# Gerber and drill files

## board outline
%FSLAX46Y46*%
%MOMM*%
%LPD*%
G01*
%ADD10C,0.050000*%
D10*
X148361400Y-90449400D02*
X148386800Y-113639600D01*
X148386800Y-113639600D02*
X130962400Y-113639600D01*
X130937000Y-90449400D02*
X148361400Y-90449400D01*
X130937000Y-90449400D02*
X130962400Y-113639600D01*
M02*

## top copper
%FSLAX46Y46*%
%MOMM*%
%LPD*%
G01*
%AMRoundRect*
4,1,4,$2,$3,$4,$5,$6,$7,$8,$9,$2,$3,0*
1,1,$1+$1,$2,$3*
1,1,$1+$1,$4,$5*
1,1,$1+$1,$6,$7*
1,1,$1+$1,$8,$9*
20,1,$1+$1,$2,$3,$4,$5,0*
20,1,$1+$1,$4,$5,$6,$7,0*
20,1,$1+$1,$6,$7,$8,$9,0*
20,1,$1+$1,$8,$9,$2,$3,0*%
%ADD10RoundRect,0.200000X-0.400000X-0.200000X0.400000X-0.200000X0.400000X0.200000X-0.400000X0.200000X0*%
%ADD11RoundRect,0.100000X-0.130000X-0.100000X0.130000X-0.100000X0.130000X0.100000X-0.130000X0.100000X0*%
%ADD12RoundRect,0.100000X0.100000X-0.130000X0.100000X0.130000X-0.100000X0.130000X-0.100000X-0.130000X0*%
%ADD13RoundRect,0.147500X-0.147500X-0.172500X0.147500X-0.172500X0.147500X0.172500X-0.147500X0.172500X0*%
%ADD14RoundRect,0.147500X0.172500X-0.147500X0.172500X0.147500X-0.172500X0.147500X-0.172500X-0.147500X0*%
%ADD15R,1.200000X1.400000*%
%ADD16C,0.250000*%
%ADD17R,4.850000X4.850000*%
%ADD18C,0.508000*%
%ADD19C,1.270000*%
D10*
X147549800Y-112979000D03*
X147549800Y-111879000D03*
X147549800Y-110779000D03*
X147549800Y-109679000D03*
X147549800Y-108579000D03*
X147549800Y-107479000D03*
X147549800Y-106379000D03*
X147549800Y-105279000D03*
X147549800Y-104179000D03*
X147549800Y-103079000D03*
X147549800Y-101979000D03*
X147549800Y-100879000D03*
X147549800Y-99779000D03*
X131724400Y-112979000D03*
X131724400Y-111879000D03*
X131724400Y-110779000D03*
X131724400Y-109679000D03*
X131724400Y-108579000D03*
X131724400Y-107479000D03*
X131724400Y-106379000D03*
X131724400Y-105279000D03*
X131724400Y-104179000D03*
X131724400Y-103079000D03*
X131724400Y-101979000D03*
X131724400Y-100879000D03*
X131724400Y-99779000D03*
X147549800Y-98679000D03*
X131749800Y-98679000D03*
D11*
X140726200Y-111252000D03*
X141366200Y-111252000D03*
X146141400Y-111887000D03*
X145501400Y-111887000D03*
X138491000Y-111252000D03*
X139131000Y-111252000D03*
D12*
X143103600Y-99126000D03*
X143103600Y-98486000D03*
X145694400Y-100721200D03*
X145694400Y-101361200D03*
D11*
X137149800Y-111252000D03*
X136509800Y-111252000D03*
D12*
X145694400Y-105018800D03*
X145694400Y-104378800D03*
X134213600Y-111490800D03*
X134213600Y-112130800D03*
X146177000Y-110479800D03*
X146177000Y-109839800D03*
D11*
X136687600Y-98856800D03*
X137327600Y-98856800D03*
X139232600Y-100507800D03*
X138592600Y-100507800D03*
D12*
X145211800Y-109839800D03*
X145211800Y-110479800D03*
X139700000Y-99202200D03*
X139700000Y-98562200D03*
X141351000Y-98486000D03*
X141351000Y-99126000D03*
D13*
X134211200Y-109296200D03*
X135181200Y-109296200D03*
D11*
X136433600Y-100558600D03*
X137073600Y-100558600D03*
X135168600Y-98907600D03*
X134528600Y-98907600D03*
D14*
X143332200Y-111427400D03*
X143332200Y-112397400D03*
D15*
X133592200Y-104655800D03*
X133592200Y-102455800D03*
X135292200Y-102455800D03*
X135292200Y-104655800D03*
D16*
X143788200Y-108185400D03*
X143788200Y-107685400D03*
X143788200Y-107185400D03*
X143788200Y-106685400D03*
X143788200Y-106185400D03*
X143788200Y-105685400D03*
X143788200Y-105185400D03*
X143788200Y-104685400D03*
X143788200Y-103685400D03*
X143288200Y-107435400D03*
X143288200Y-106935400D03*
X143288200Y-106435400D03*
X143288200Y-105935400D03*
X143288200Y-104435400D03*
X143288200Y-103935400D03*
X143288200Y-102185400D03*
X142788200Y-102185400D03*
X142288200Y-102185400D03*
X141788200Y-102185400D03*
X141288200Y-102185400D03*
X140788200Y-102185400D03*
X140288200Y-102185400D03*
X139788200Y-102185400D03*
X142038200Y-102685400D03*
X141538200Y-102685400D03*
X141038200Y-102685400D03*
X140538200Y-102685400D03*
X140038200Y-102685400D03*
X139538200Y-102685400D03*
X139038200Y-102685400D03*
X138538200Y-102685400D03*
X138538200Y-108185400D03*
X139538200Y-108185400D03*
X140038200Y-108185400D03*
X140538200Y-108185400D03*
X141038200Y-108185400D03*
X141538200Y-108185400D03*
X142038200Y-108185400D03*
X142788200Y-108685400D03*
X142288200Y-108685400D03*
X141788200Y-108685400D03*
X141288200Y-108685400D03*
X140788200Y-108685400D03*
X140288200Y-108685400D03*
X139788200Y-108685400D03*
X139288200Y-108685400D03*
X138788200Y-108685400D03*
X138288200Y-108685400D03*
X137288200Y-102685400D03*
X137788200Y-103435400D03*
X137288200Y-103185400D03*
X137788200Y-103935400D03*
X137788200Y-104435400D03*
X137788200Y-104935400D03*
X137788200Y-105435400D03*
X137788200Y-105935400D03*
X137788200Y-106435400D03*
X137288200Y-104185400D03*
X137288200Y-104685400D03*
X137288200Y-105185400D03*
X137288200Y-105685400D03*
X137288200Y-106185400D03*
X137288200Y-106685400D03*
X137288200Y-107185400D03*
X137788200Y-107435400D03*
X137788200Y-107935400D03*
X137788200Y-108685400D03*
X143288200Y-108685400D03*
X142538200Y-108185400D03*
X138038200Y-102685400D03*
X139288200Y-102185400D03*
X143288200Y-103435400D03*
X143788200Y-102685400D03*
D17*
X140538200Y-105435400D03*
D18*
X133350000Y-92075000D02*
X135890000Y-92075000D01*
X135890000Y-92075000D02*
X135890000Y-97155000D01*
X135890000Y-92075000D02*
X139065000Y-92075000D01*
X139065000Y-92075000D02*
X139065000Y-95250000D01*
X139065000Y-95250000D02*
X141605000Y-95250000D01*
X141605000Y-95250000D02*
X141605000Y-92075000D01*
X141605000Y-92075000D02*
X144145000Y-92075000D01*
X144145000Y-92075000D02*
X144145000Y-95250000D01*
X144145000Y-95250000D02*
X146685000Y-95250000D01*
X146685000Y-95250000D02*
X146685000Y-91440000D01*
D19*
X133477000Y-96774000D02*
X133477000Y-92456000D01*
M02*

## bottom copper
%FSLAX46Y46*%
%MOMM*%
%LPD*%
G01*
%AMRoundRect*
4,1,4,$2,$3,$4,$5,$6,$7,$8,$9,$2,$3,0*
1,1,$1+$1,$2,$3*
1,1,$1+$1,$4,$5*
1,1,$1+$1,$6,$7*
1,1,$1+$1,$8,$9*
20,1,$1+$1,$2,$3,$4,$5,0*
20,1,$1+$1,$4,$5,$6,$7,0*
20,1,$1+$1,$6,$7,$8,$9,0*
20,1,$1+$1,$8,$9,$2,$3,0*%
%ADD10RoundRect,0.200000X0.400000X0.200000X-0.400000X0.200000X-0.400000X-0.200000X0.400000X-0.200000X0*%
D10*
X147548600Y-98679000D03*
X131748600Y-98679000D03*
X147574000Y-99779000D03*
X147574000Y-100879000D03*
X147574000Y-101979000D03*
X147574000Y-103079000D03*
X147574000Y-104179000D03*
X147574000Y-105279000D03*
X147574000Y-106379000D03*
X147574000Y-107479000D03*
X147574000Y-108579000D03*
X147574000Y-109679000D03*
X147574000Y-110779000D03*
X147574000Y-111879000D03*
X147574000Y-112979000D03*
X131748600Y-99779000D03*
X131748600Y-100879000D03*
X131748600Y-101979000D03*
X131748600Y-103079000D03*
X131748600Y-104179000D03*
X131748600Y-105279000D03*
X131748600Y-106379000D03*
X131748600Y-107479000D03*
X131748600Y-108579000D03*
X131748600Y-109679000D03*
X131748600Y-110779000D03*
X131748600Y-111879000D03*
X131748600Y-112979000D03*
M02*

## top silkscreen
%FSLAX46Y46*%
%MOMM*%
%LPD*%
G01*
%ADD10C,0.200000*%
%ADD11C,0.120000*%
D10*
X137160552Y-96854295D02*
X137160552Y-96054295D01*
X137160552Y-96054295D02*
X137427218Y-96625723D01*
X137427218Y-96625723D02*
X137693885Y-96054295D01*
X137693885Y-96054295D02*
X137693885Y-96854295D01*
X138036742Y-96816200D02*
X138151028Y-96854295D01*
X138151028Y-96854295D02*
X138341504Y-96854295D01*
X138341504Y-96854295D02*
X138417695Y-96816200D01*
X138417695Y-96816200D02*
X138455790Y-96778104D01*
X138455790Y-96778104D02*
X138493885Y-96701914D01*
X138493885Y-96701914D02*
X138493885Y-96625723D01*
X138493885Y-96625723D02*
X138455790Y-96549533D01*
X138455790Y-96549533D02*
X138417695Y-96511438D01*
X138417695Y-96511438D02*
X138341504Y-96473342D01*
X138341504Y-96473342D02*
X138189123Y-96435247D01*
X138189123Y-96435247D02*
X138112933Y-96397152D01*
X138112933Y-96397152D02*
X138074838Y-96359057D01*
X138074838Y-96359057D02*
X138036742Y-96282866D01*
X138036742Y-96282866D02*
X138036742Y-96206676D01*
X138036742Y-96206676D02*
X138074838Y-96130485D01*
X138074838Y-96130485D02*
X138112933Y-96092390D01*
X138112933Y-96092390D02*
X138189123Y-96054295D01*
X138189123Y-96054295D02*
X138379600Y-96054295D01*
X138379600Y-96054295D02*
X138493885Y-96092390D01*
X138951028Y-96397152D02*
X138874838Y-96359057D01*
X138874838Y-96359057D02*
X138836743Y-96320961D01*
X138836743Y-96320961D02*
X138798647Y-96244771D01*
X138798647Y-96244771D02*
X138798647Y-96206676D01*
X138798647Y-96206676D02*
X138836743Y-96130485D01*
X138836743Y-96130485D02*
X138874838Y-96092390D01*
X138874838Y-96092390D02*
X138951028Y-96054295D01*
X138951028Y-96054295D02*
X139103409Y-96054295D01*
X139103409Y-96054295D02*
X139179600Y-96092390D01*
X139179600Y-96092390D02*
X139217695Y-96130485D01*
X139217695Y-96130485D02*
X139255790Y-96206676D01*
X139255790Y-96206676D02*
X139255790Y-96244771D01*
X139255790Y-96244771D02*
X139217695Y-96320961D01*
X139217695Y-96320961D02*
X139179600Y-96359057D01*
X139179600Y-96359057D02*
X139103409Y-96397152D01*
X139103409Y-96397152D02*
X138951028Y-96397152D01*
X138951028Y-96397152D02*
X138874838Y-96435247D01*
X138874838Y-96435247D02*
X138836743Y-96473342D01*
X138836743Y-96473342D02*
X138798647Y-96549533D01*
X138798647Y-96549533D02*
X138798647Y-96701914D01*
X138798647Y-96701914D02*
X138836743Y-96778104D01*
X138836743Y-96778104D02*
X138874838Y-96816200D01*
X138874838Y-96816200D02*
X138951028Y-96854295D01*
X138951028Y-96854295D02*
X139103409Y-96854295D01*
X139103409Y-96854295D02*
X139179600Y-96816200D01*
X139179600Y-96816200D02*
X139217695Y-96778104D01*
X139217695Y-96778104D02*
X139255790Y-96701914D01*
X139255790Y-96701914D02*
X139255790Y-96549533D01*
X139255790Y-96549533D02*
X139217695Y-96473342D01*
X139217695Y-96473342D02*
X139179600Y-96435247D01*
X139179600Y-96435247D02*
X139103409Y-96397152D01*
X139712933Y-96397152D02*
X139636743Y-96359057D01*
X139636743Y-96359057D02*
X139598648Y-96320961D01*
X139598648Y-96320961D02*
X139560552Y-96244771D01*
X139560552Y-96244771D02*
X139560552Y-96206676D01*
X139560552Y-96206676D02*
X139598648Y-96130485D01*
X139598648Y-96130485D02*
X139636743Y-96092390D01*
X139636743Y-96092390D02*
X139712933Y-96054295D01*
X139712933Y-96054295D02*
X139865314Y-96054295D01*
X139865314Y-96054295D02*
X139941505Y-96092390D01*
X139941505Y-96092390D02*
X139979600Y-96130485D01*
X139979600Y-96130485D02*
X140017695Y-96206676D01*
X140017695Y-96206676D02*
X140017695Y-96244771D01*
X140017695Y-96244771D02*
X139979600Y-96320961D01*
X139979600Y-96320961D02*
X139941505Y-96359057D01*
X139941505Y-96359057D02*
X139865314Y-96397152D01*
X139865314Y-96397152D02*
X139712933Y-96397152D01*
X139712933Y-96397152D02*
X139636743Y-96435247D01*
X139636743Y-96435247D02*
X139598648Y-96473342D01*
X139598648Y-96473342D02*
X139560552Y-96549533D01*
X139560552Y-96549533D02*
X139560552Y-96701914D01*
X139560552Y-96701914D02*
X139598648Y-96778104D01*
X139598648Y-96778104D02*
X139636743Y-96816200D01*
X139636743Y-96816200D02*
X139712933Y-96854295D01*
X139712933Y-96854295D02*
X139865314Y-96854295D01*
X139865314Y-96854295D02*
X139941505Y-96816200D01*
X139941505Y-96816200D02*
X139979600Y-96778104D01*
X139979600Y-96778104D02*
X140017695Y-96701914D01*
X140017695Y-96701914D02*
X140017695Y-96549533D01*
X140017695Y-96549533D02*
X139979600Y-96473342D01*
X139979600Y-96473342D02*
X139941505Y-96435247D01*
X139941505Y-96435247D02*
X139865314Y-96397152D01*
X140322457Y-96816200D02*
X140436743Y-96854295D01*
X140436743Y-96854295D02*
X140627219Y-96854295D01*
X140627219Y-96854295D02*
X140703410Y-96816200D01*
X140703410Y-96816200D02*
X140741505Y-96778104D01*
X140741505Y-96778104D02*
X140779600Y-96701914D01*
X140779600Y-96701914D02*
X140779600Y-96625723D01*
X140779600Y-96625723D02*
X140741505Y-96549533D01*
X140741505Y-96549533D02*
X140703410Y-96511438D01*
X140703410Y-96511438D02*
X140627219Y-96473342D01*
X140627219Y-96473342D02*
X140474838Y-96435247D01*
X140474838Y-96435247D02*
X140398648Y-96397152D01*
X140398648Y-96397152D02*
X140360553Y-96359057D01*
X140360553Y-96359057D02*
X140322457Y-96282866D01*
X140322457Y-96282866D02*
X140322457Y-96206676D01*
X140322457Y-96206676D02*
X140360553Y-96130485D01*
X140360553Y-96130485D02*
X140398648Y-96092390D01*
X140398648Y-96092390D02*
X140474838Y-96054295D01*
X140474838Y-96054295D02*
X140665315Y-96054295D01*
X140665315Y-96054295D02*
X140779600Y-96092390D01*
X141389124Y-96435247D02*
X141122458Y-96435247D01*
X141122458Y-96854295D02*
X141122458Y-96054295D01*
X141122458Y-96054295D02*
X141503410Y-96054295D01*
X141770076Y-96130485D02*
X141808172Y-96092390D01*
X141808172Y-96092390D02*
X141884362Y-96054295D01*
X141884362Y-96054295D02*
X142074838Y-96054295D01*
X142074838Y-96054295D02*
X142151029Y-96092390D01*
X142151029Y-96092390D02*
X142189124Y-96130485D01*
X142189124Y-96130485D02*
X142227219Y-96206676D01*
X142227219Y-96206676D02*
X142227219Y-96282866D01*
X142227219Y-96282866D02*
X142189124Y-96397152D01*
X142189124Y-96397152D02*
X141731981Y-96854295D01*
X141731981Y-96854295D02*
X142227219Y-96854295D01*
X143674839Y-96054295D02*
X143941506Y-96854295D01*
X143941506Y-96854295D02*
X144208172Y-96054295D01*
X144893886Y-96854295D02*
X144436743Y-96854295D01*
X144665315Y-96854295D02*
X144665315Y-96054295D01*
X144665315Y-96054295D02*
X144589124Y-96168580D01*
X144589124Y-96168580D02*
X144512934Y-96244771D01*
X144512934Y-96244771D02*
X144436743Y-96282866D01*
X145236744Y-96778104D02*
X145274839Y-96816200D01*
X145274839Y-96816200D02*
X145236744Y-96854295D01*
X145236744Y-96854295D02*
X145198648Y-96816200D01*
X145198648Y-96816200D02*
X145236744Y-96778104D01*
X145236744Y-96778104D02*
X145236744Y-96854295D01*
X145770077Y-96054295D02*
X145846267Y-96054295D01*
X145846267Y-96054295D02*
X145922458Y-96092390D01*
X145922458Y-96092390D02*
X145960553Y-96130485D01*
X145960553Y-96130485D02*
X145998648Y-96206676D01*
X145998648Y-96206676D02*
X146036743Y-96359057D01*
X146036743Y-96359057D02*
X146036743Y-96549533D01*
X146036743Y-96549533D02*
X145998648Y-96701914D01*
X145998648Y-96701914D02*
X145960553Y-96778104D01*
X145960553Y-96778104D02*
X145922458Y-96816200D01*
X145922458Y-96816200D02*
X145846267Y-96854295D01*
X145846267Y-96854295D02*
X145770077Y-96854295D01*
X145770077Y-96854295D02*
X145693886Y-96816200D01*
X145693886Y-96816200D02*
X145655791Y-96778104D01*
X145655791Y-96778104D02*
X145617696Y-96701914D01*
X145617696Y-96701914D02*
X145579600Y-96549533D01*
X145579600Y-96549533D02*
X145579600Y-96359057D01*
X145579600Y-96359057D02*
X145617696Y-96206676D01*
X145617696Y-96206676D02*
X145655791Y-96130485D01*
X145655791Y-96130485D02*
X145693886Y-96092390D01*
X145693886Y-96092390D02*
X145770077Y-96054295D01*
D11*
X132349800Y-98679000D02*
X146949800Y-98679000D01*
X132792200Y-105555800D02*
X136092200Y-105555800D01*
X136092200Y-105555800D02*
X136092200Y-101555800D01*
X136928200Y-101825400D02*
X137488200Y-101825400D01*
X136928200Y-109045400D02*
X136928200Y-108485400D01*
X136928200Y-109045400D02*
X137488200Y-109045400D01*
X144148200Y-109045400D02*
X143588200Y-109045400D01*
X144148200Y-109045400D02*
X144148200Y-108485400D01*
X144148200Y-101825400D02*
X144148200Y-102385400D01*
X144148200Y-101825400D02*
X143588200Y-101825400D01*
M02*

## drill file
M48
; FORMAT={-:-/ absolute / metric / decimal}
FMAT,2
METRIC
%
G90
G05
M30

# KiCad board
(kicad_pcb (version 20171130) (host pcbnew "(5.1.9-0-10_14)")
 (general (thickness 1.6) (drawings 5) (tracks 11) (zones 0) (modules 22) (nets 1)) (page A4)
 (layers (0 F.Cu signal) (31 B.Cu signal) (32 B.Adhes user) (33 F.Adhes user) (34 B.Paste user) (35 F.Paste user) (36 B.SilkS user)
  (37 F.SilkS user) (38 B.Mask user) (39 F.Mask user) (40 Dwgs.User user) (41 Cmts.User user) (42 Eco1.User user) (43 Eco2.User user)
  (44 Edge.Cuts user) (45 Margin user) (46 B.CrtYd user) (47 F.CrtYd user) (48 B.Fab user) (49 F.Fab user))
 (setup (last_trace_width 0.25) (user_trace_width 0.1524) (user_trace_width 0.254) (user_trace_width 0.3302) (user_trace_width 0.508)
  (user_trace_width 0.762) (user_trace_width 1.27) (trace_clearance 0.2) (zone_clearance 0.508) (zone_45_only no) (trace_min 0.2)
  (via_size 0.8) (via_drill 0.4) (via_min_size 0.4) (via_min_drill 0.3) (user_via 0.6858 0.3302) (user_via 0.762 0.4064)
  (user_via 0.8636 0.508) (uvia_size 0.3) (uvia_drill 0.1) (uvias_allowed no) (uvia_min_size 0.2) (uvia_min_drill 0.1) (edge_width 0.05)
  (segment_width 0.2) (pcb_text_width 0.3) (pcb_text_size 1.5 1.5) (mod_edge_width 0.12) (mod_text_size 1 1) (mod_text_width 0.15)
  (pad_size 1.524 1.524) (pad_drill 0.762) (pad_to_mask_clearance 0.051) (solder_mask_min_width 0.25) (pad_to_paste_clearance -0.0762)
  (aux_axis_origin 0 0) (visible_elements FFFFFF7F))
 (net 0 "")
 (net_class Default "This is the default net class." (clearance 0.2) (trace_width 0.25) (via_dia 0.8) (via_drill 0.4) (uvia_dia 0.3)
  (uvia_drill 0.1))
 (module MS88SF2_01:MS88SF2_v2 (layer B.Cu) (at 147.5486 98.679 180)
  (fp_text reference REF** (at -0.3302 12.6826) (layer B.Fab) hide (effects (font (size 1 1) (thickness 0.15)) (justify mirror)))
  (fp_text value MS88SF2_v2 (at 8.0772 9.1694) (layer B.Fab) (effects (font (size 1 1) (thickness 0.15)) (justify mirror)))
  (pad 1 smd roundrect (at 0 0 180) (size 1.2 0.8) (layers B.Cu B.Paste B.Mask) (roundrect_rratio 0.25))
  (pad 1 smd roundrect (at 15.8 0 180) (size 1.2 0.8) (layers B.Cu B.Paste B.Mask) (roundrect_rratio 0.25))
  (pad 2 smd roundrect (at -0.0254 -1.1 180) (size 1.2 0.8) (layers B.Cu B.Paste B.Mask) (roundrect_rratio 0.25))
  (pad 3 smd roundrect (at -0.0254 -2.2 180) (size 1.2 0.8) (layers B.Cu B.Paste B.Mask) (roundrect_rratio 0.25))
  (pad 4 smd roundrect (at -0.0254 -3.3 180) (size 1.2 0.8) (layers B.Cu B.Paste B.Mask) (roundrect_rratio 0.25))
  (pad 5 smd roundrect (at -0.0254 -4.4 180) (size 1.2 0.8) (layers B.Cu B.Paste B.Mask) (roundrect_rratio 0.25))
  (pad 6 smd roundrect (at -0.0254 -5.5 180) (size 1.2 0.8) (layers B.Cu B.Paste B.Mask) (roundrect_rratio 0.25))
  (pad 7 smd roundrect (at -0.0254 -6.6 180) (size 1.2 0.8) (layers B.Cu B.Paste B.Mask) (roundrect_rratio 0.25))
  (pad 8 smd roundrect (at -0.0254 -7.7 180) (size 1.2 0.8) (layers B.Cu B.Paste B.Mask) (roundrect_rratio 0.25))
  (pad 9 smd roundrect (at -0.0254 -8.8 180) (size 1.2 0.8) (layers B.Cu B.Paste B.Mask) (roundrect_rratio 0.25))
  (pad 10 smd roundrect (at -0.0254 -9.9 180) (size 1.2 0.8) (layers B.Cu B.Paste B.Mask) (roundrect_rratio 0.25))
  (pad 11 smd roundrect (at -0.0254 -11 180) (size 1.2 0.8) (layers B.Cu B.Paste B.Mask) (roundrect_rratio 0.25))
  (pad 12 smd roundrect (at -0.0254 -12.1 180) (size 1.2 0.8) (layers B.Cu B.Paste B.Mask) (roundrect_rratio 0.25))
  (pad 13 smd roundrect (at -0.0254 -13.2 180) (size 1.2 0.8) (layers B.Cu B.Paste B.Mask) (roundrect_rratio 0.25))
  (pad 14 smd roundrect (at -0.0254 -14.3 180) (size 1.2 0.8) (layers B.Cu B.Paste B.Mask) (roundrect_rratio 0.25))
  (pad 2 smd roundrect (at 15.8 -1.1 180) (size 1.2 0.8) (layers B.Cu B.Paste B.Mask) (roundrect_rratio 0.25))
  (pad 3 smd roundrect (at 15.8 -2.2 180) (size 1.2 0.8) (layers B.Cu B.Paste B.Mask) (roundrect_rratio 0.25))
  (pad 4 smd roundrect (at 15.8 -3.3 180) (size 1.2 0.8) (layers B.Cu B.Paste B.Mask) (roundrect_rratio 0.25))
  (pad 5 smd roundrect (at 15.8 -4.4 180) (size 1.2 0.8) (layers B.Cu B.Paste B.Mask) (roundrect_rratio 0.25))
  (pad 6 smd roundrect (at 15.8 -5.5 180) (size 1.2 0.8) (layers B.Cu B.Paste B.Mask) (roundrect_rratio 0.25))
  (pad 7 smd roundrect (at 15.8 -6.6 180) (size 1.2 0.8) (layers B.Cu B.Paste B.Mask) (roundrect_rratio 0.25))
  (pad 8 smd roundrect (at 15.8 -7.7 180) (size 1.2 0.8) (layers B.Cu B.Paste B.Mask) (roundrect_rratio 0.25))
  (pad 9 smd roundrect (at 15.8 -8.8 180) (size 1.2 0.8) (layers B.Cu B.Paste B.Mask) (roundrect_rratio 0.25))
  (pad 10 smd roundrect (at 15.8 -9.9 180) (size 1.2 0.8) (layers B.Cu B.Paste B.Mask) (roundrect_rratio 0.25))
  (pad 11 smd roundrect (at 15.8 -11 180) (size 1.2 0.8) (layers B.Cu B.Paste B.Mask) (roundrect_rratio 0.25))
  (pad 12 smd roundrect (at 15.8 -12.1 180) (size 1.2 0.8) (layers B.Cu B.Paste B.Mask) (roundrect_rratio 0.25))
  (pad 13 smd roundrect (at 15.8 -13.2 180) (size 1.2 0.8) (layers B.Cu B.Paste B.Mask) (roundrect_rratio 0.25))
  (pad 14 smd roundrect (at 15.8 -14.3 180) (size 1.2 0.8) (layers B.Cu B.Paste B.Mask) (roundrect_rratio 0.25)))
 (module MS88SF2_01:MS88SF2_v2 (layer F.Cu) (at 131.7498 98.679)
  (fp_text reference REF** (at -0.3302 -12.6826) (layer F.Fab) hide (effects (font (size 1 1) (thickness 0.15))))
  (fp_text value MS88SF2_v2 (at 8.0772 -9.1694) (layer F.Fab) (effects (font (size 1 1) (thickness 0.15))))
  (fp_line (start 0.6 0) (end 15.2 0) (layer F.SilkS) (width 0.12))
  (pad 14 smd roundrect (at 15.8 14.3) (size 1.2 0.8) (layers F.Cu F.Paste F.Mask) (roundrect_rratio 0.25))
  (pad 13 smd roundrect (at 15.8 13.2) (size 1.2 0.8) (layers F.Cu F.Paste F.Mask) (roundrect_rratio 0.25))
  (pad 12 smd roundrect (at 15.8 12.1) (size 1.2 0.8) (layers F.Cu F.Paste F.Mask) (roundrect_rratio 0.25))
  (pad 11 smd roundrect (at 15.8 11) (size 1.2 0.8) (layers F.Cu F.Paste F.Mask) (roundrect_rratio 0.25))
  (pad 10 smd roundrect (at 15.8 9.9) (size 1.2 0.8) (layers F.Cu F.Paste F.Mask) (roundrect_rratio 0.25))
  (pad 9 smd roundrect (at 15.8 8.8) (size 1.2 0.8) (layers F.Cu F.Paste F.Mask) (roundrect_rratio 0.25))
  (pad 8 smd roundrect (at 15.8 7.7) (size 1.2 0.8) (layers F.Cu F.Paste F.Mask) (roundrect_rratio 0.25))
  (pad 7 smd roundrect (at 15.8 6.6) (size 1.2 0.8) (layers F.Cu F.Paste F.Mask) (roundrect_rratio 0.25))
  (pad 6 smd roundrect (at 15.8 5.5) (size 1.2 0.8) (layers F.Cu F.Paste F.Mask) (roundrect_rratio 0.25))
  (pad 5 smd roundrect (at 15.8 4.4) (size 1.2 0.8) (layers F.Cu F.Paste F.Mask) (roundrect_rratio 0.25))
  (pad 4 smd roundrect (at 15.8 3.3) (size 1.2 0.8) (layers F.Cu F.Paste F.Mask) (roundrect_rratio 0.25))
  (pad 3 smd roundrect (at 15.8 2.2) (size 1.2 0.8) (layers F.Cu F.Paste F.Mask) (roundrect_rratio 0.25))
  (pad 2 smd roundrect (at 15.8 1.1) (size 1.2 0.8) (layers F.Cu F.Paste F.Mask) (roundrect_rratio 0.25))
  (pad 14 smd roundrect (at -0.0254 14.3) (size 1.2 0.8) (layers F.Cu F.Paste F.Mask) (roundrect_rratio 0.25))
  (pad 13 smd roundrect (at -0.0254 13.2) (size 1.2 0.8) (layers F.Cu F.Paste F.Mask) (roundrect_rratio 0.25))
  (pad 12 smd roundrect (at -0.0254 12.1) (size 1.2 0.8) (layers F.Cu F.Paste F.Mask) (roundrect_rratio 0.25))
  (pad 11 smd roundrect (at -0.0254 11) (size 1.2 0.8) (layers F.Cu F.Paste F.Mask) (roundrect_rratio 0.25))
  (pad 10 smd roundrect (at -0.0254 9.9) (size 1.2 0.8) (layers F.Cu F.Paste F.Mask) (roundrect_rratio 0.25))
  (pad 9 smd roundrect (at -0.0254 8.8) (size 1.2 0.8) (layers F.Cu F.Paste F.Mask) (roundrect_rratio 0.25))
  (pad 8 smd roundrect (at -0.0254 7.7) (size 1.2 0.8) (layers F.Cu F.Paste F.Mask) (roundrect_rratio 0.25))
  (pad 7 smd roundrect (at -0.0254 6.6) (size 1.2 0.8) (layers F.Cu F.Paste F.Mask) (roundrect_rratio 0.25))
  (pad 6 smd roundrect (at -0.0254 5.5) (size 1.2 0.8) (layers F.Cu F.Paste F.Mask) (roundrect_rratio 0.25))
  (pad 5 smd roundrect (at -0.0254 4.4) (size 1.2 0.8) (layers F.Cu F.Paste F.Mask) (roundrect_rratio 0.25))
  (pad 4 smd roundrect (at -0.0254 3.3) (size 1.2 0.8) (layers F.Cu F.Paste F.Mask) (roundrect_rratio 0.25))
  (pad 3 smd roundrect (at -0.0254 2.2) (size 1.2 0.8) (layers F.Cu F.Paste F.Mask) (roundrect_rratio 0.25))
  (pad 2 smd roundrect (at -0.0254 1.1) (size 1.2 0.8) (layers F.Cu F.Paste F.Mask) (roundrect_rratio 0.25))
  (pad 1 smd roundrect (at 15.8 0) (size 1.2 0.8) (layers F.Cu F.Paste F.Mask) (roundrect_rratio 0.25))
  (pad 1 smd roundrect (at 0 0) (size 1.2 0.8) (layers F.Cu F.Paste F.Mask) (roundrect_rratio 0.25)))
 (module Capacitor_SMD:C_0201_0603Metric (layer F.Cu) (at 141.0462 111.252)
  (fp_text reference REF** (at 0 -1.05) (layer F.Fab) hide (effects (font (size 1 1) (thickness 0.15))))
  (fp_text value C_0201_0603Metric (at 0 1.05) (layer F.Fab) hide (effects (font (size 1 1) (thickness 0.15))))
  (pad "" smd roundrect (at -0.345 0) (size 0.318 0.36) (layers F.Paste) (roundrect_rratio 0.25))
  (pad "" smd roundrect (at 0.345 0) (size 0.318 0.36) (layers F.Paste) (roundrect_rratio 0.25))
  (pad 1 smd roundrect (at -0.32 0) (size 0.46 0.4) (layers F.Cu F.Mask) (roundrect_rratio 0.25))
  (pad 2 smd roundrect (at 0.32 0) (size 0.46 0.4) (layers F.Cu F.Mask) (roundrect_rratio 0.25)))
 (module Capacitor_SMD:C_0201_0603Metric (layer F.Cu) (at 145.8214 111.887)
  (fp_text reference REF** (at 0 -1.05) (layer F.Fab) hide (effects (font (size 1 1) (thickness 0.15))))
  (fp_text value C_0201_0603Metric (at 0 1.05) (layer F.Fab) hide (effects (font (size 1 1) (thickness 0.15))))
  (pad 2 smd roundrect (at 0.32 0) (size 0.46 0.4) (layers F.Cu F.Mask) (roundrect_rratio 0.25))
  (pad 1 smd roundrect (at -0.32 0) (size 0.46 0.4) (layers F.Cu F.Mask) (roundrect_rratio 0.25))
  (pad "" smd roundrect (at 0.345 0) (size 0.318 0.36) (layers F.Paste) (roundrect_rratio 0.25))
  (pad "" smd roundrect (at -0.345 0) (size 0.318 0.36) (layers F.Paste) (roundrect_rratio 0.25)))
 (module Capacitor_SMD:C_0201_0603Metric (layer F.Cu) (at 138.811 111.252)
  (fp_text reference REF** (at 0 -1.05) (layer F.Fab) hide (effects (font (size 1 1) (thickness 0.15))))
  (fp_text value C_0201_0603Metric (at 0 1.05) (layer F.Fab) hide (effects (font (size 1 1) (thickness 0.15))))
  (pad "" smd roundrect (at -0.345 0) (size 0.318 0.36) (layers F.Paste) (roundrect_rratio 0.25))
  (pad "" smd roundrect (at 0.345 0) (size 0.318 0.36) (layers F.Paste) (roundrect_rratio 0.25))
  (pad 1 smd roundrect (at -0.32 0) (size 0.46 0.4) (layers F.Cu F.Mask) (roundrect_rratio 0.25))
  (pad 2 smd roundrect (at 0.32 0) (size 0.46 0.4) (layers F.Cu F.Mask) (roundrect_rratio 0.25)))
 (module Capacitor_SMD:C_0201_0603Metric (layer F.Cu) (at 143.1036 98.806 90)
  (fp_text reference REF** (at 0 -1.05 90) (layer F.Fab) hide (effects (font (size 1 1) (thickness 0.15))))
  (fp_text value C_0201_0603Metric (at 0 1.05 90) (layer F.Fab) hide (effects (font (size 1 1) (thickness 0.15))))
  (pad "" smd roundrect (at -0.345 0 90) (size 0.318 0.36) (layers F.Paste) (roundrect_rratio 0.25))
  (pad "" smd roundrect (at 0.345 0 90) (size 0.318 0.36) (layers F.Paste) (roundrect_rratio 0.25))
  (pad 1 smd roundrect (at -0.32 0 90) (size 0.46 0.4) (layers F.Cu F.Mask) (roundrect_rratio 0.25))
  (pad 2 smd roundrect (at 0.32 0 90) (size 0.46 0.4) (layers F.Cu F.Mask) (roundrect_rratio 0.25)))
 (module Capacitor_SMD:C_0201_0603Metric (layer F.Cu) (at 145.6944 101.0412 90)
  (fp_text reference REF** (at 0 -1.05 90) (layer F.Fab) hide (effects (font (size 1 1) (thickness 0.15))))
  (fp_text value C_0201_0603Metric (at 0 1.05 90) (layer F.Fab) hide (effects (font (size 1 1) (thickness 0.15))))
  (pad 2 smd roundrect (at 0.32 0 90) (size 0.46 0.4) (layers F.Cu F.Mask) (roundrect_rratio 0.25))
  (pad 1 smd roundrect (at -0.32 0 90) (size 0.46 0.4) (layers F.Cu F.Mask) (roundrect_rratio 0.25))
  (pad "" smd roundrect (at 0.345 0 90) (size 0.318 0.36) (layers F.Paste) (roundrect_rratio 0.25))
  (pad "" smd roundrect (at -0.345 0 90) (size 0.318 0.36) (layers F.Paste) (roundrect_rratio 0.25)))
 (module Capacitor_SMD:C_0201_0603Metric (layer F.Cu) (at 136.8298 111.252)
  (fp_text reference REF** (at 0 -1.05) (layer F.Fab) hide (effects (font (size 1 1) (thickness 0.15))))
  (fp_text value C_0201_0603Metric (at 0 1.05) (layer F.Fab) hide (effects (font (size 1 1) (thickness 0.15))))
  (pad 2 smd roundrect (at 0.32 0) (size 0.46 0.4) (layers F.Cu F.Mask) (roundrect_rratio 0.25))
  (pad 1 smd roundrect (at -0.32 0) (size 0.46 0.4) (layers F.Cu F.Mask) (roundrect_rratio 0.25))
  (pad "" smd roundrect (at 0.345 0) (size 0.318 0.36) (layers F.Paste) (roundrect_rratio 0.25))
  (pad "" smd roundrect (at -0.345 0) (size 0.318 0.36) (layers F.Paste) (roundrect_rratio 0.25)))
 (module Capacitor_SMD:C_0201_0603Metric (layer F.Cu) (at 145.6944 104.6988 90)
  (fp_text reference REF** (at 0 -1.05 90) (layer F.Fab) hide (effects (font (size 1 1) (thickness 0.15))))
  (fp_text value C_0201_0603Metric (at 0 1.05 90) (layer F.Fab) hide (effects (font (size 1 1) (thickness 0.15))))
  (pad "" smd roundrect (at -0.345 0 90) (size 0.318 0.36) (layers F.Paste) (roundrect_rratio 0.25))
  (pad "" smd roundrect (at 0.345 0 90) (size 0.318 0.36) (layers F.Paste) (roundrect_rratio 0.25))
  (pad 1 smd roundrect (at -0.32 0 90) (size 0.46 0.4) (layers F.Cu F.Mask) (roundrect_rratio 0.25))
  (pad 2 smd roundrect (at 0.32 0 90) (size 0.46 0.4) (layers F.Cu F.Mask) (roundrect_rratio 0.25)))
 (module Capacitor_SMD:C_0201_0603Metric (layer F.Cu) (at 134.2136 111.8108 90)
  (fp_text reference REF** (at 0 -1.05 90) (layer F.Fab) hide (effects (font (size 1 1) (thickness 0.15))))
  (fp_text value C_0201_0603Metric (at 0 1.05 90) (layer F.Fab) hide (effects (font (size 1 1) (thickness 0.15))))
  (pad 2 smd roundrect (at 0.32 0 90) (size 0.46 0.4) (layers F.Cu F.Mask) (roundrect_rratio 0.25))
  (pad 1 smd roundrect (at -0.32 0 90) (size 0.46 0.4) (layers F.Cu F.Mask) (roundrect_rratio 0.25))
  (pad "" smd roundrect (at 0.345 0 90) (size 0.318 0.36) (layers F.Paste) (roundrect_rratio 0.25))
  (pad "" smd roundrect (at -0.345 0 90) (size 0.318 0.36) (layers F.Paste) (roundrect_rratio 0.25)))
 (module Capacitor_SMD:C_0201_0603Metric (layer F.Cu) (at 146.177 110.1598 90)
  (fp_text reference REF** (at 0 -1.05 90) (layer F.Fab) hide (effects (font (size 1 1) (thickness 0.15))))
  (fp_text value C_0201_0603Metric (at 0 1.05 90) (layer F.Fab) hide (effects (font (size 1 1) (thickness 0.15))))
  (pad "" smd roundrect (at -0.345 0 90) (size 0.318 0.36) (layers F.Paste) (roundrect_rratio 0.25))
  (pad "" smd roundrect (at 0.345 0 90) (size 0.318 0.36) (layers F.Paste) (roundrect_rratio 0.25))
  (pad 1 smd roundrect (at -0.32 0 90) (size 0.46 0.4) (layers F.Cu F.Mask) (roundrect_rratio 0.25))
  (pad 2 smd roundrect (at 0.32 0 90) (size 0.46 0.4) (layers F.Cu F.Mask) (roundrect_rratio 0.25)))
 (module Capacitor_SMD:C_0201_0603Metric (layer F.Cu) (at 137.0076 98.8568)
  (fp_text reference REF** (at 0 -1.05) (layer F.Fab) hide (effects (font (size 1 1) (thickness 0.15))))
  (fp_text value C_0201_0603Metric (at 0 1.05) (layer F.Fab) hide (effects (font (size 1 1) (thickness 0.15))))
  (pad "" smd roundrect (at -0.345 0) (size 0.318 0.36) (layers F.Paste) (roundrect_rratio 0.25))
  (pad "" smd roundrect (at 0.345 0) (size 0.318 0.36) (layers F.Paste) (roundrect_rratio 0.25))
  (pad 1 smd roundrect (at -0.32 0) (size 0.46 0.4) (layers F.Cu F.Mask) (roundrect_rratio 0.25))
  (pad 2 smd roundrect (at 0.32 0) (size 0.46 0.4) (layers F.Cu F.Mask) (roundrect_rratio 0.25)))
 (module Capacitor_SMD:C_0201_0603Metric (layer F.Cu) (at 138.9126 100.5078)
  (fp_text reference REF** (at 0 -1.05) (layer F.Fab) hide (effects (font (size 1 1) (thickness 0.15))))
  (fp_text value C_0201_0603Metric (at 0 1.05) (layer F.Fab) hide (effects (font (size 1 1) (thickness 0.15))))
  (pad 2 smd roundrect (at 0.32 0) (size 0.46 0.4) (layers F.Cu F.Mask) (roundrect_rratio 0.25))
  (pad 1 smd roundrect (at -0.32 0) (size 0.46 0.4) (layers F.Cu F.Mask) (roundrect_rratio 0.25))
  (pad "" smd roundrect (at 0.345 0) (size 0.318 0.36) (layers F.Paste) (roundrect_rratio 0.25))
  (pad "" smd roundrect (at -0.345 0) (size 0.318 0.36) (layers F.Paste) (roundrect_rratio 0.25)))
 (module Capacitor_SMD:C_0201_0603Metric (layer F.Cu) (at 145.2118 110.1598 90)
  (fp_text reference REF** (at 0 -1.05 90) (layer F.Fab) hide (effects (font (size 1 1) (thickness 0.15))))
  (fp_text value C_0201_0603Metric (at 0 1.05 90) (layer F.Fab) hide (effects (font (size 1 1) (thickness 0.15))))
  (pad 2 smd roundrect (at 0.32 0 90) (size 0.46 0.4) (layers F.Cu F.Mask) (roundrect_rratio 0.25))
  (pad 1 smd roundrect (at -0.32 0 90) (size 0.46 0.4) (layers F.Cu F.Mask) (roundrect_rratio 0.25))
  (pad "" smd roundrect (at 0.345 0 90) (size 0.318 0.36) (layers F.Paste) (roundrect_rratio 0.25))
  (pad "" smd roundrect (at -0.345 0 90) (size 0.318 0.36) (layers F.Paste) (roundrect_rratio 0.25)))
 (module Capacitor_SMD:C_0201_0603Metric (layer F.Cu) (at 139.7 98.8822 90)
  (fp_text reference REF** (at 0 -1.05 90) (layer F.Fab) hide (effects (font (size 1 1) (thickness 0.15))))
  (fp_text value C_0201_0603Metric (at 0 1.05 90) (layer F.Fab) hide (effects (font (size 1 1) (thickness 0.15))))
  (pad "" smd roundrect (at -0.345 0 90) (size 0.318 0.36) (layers F.Paste) (roundrect_rratio 0.25))
  (pad "" smd roundrect (at 0.345 0 90) (size 0.318 0.36) (layers F.Paste) (roundrect_rratio 0.25))
  (pad 1 smd roundrect (at -0.32 0 90) (size 0.46 0.4) (layers F.Cu F.Mask) (roundrect_rratio 0.25))
  (pad 2 smd roundrect (at 0.32 0 90) (size 0.46 0.4) (layers F.Cu F.Mask) (roundrect_rratio 0.25)))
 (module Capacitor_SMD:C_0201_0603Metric (layer F.Cu) (at 141.351 98.806 90)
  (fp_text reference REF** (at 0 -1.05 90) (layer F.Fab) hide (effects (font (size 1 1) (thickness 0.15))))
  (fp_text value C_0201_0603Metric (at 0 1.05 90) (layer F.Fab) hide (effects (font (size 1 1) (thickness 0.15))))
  (pad 2 smd roundrect (at 0.32 0 90) (size 0.46 0.4) (layers F.Cu F.Mask) (roundrect_rratio 0.25))
  (pad 1 smd roundrect (at -0.32 0 90) (size 0.46 0.4) (layers F.Cu F.Mask) (roundrect_rratio 0.25))
  (pad "" smd roundrect (at 0.345 0 90) (size 0.318 0.36) (layers F.Paste) (roundrect_rratio 0.25))
  (pad "" smd roundrect (at -0.345 0 90) (size 0.318 0.36) (layers F.Paste) (roundrect_rratio 0.25)))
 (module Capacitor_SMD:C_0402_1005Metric (layer F.Cu) (at 134.6962 109.2962)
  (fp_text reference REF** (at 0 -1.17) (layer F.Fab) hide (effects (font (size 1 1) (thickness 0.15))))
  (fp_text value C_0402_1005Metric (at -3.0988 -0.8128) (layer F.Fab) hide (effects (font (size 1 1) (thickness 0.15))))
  (pad 1 smd roundrect (at -0.485 0) (size 0.59 0.64) (layers F.Cu F.Paste F.Mask) (roundrect_rratio 0.25))
  (pad 2 smd roundrect (at 0.485 0) (size 0.59 0.64) (layers F.Cu F.Paste F.Mask) (roundrect_rratio 0.25)))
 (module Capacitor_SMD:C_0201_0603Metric (layer F.Cu) (at 136.7536 100.5586)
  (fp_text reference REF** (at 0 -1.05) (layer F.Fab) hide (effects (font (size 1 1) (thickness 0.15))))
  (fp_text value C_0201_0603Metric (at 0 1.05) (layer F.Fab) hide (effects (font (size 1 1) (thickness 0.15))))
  (pad "" smd roundrect (at -0.345 0) (size 0.318 0.36) (layers F.Paste) (roundrect_rratio 0.25))
  (pad "" smd roundrect (at 0.345 0) (size 0.318 0.36) (layers F.Paste) (roundrect_rratio 0.25))
  (pad 1 smd roundrect (at -0.32 0) (size 0.46 0.4) (layers F.Cu F.Mask) (roundrect_rratio 0.25))
  (pad 2 smd roundrect (at 0.32 0) (size 0.46 0.4) (layers F.Cu F.Mask) (roundrect_rratio 0.25)))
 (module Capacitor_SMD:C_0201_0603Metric (layer F.Cu) (at 134.8486 98.9076)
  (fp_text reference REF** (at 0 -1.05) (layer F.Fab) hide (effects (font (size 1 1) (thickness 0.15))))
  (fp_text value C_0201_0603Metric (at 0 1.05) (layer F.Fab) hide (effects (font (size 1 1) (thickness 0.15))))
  (pad 2 smd roundrect (at 0.32 0) (size 0.46 0.4) (layers F.Cu F.Mask) (roundrect_rratio 0.25))
  (pad 1 smd roundrect (at -0.32 0) (size 0.46 0.4) (layers F.Cu F.Mask) (roundrect_rratio 0.25))
  (pad "" smd roundrect (at 0.345 0) (size 0.318 0.36) (layers F.Paste) (roundrect_rratio 0.25))
  (pad "" smd roundrect (at -0.345 0) (size 0.318 0.36) (layers F.Paste) (roundrect_rratio 0.25)))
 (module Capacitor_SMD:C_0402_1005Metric (layer F.Cu) (at 143.3322 111.9124 90)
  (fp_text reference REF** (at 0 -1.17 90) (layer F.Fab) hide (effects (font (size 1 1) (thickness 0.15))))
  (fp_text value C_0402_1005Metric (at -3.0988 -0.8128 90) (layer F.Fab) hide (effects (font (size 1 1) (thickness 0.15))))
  (pad 2 smd roundrect (at 0.485 0 90) (size 0.59 0.64) (layers F.Cu F.Paste F.Mask) (roundrect_rratio 0.25))
  (pad 1 smd roundrect (at -0.485 0 90) (size 0.59 0.64) (layers F.Cu F.Paste F.Mask) (roundrect_rratio 0.25)))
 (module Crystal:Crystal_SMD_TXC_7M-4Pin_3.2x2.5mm (layer F.Cu) (at 134.4422 103.5558 90)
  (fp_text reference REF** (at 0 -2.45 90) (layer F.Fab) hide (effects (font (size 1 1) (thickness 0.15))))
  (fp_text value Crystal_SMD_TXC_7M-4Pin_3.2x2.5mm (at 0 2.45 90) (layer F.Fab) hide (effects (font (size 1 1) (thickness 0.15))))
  (fp_line (start -2 -1.65) (end -2 1.65) (layer F.SilkS) (width 0.12))
  (fp_line (start -2 1.65) (end 2 1.65) (layer F.SilkS) (width 0.12))
  (pad 4 smd rect (at -1.1 -0.85 90) (size 1.4 1.2) (layers F.Cu F.Paste F.Mask))
  (pad 3 smd rect (at 1.1 -0.85 90) (size 1.4 1.2) (layers F.Cu F.Paste F.Mask))
  (pad 2 smd rect (at 1.1 0.85 90) (size 1.4 1.2) (layers F.Cu F.Paste F.Mask))
  (pad 1 smd rect (at -1.1 0.85 90) (size 1.4 1.2) (layers F.Cu F.Paste F.Mask)))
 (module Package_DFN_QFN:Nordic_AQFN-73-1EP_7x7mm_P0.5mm (layer F.Cu) (at 140.5382 105.4354)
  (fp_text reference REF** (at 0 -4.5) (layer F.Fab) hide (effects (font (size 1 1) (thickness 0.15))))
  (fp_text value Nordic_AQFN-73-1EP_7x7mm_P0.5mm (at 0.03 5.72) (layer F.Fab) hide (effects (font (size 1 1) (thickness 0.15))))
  (fp_line (start -3.61 -3.61) (end -3.05 -3.61) (layer F.SilkS) (width 0.12))
  (fp_line (start -3.61 3.61) (end -3.61 3.05) (layer F.SilkS) (width 0.12))
  (fp_line (start -3.61 3.61) (end -3.05 3.61) (layer F.SilkS) (width 0.12))
  (fp_line (start 3.61 3.61) (end 3.05 3.61) (layer F.SilkS) (width 0.12))
  (fp_line (start 3.61 3.61) (end 3.61 3.05) (layer F.SilkS) (width 0.12))
  (fp_line (start 3.61 -3.61) (end 3.61 -3.05) (layer F.SilkS) (width 0.12))
  (fp_line (start 3.61 -3.61) (end 3.05 -3.61) (layer F.SilkS) (width 0.12))
  (pad AC24 smd circle (at 3.25 2.75 180) (size 0.25 0.25) (layers F.Cu F.Paste F.Mask))
  (pad AA24 smd circle (at 3.25 2.25 180) (size 0.25 0.25) (layers F.Cu F.Paste F.Mask))
  (pad W24 smd circle (at 3.25 1.75 180) (size 0.25 0.25) (layers F.Cu F.Paste F.Mask))
  (pad U24 smd circle (at 3.25 1.25 180) (size 0.25 0.25) (layers F.Cu F.Paste F.Mask))
  (pad R24 smd circle (at 3.25 0.75 180) (size 0.25 0.25) (layers F.Cu F.Paste F.Mask))
  (pad N24 smd circle (at 3.25 0.25 180) (size 0.25 0.25) (layers F.Cu F.Paste F.Mask))
  (pad L24 smd circle (at 3.25 -0.25 180) (size 0.25 0.25) (layers F.Cu F.Paste F.Mask))
  (pad J24 smd circle (at 3.25 -0.75 180) (size 0.25 0.25) (layers F.Cu F.Paste F.Mask))
  (pad E24 smd circle (at 3.25 -1.75 180) (size 0.25 0.25) (layers F.Cu F.Paste F.Mask))
  (pad Y23 smd circle (at 2.75 2 180) (size 0.25 0.25) (layers F.Cu F.Paste F.Mask))
  (pad V23 smd circle (at 2.75 1.5 180) (size 0.25 0.25) (layers F.Cu F.Paste F.Mask))
  (pad T23 smd circle (at 2.75 1 180) (size 0.25 0.25) (layers F.Cu F.Paste F.Mask))
  (pad P23 smd circle (at 2.75 0.5 180) (size 0.25 0.25) (layers F.Cu F.Paste F.Mask))
  (pad H23 smd circle (at 2.75 -1 180) (size 0.25 0.25) (layers F.Cu F.Paste F.Mask))
  (pad F23 smd circle (at 2.75 -1.5 180) (size 0.25 0.25) (layers F.Cu F.Paste F.Mask))
  (pad A23 smd circle (at 2.75 -3.25 180) (size 0.25 0.25) (layers F.Cu F.Paste F.Mask))
  (pad A22 smd circle (at 2.25 -3.25 180) (size 0.25 0.25) (layers F.Cu F.Paste F.Mask))
  (pad A20 smd circle (at 1.75 -3.25 180) (size 0.25 0.25) (layers F.Cu F.Paste F.Mask))
  (pad A18 smd circle (at 1.25 -3.25 180) (size 0.25 0.25) (layers F.Cu F.Paste F.Mask))
  (pad A16 smd circle (at 0.75 -3.25 180) (size 0.25 0.25) (layers F.Cu F.Paste F.Mask))
  (pad A14 smd circle (at 0.25 -3.25 180) (size 0.25 0.25) (layers F.Cu F.Paste F.Mask))
  (pad A12 smd circle (at -0.25 -3.25 180) (size 0.25 0.25) (layers F.Cu F.Paste F.Mask))
  (pad A10 smd circle (at -0.75 -3.25 180) (size 0.25 0.25) (layers F.Cu F.Paste F.Mask))
  (pad B19 smd circle (at 1.5 -2.75 180) (size 0.25 0.25) (layers F.Cu F.Paste F.Mask))
  (pad B17 smd circle (at 1 -2.75 180) (size 0.25 0.25) (layers F.Cu F.Paste F.Mask))
  (pad B15 smd circle (at 0.5 -2.75 180) (size 0.25 0.25) (layers F.Cu F.Paste F.Mask))
  (pad B13 smd circle (at 0 -2.75 180) (size 0.25 0.25) (layers F.Cu F.Paste F.Mask))
  (pad B11 smd circle (at -0.5 -2.75 180) (size 0.25 0.25) (layers F.Cu F.Paste F.Mask))
  (pad B9 smd circle (at -1 -2.75 180) (size 0.25 0.25) (layers F.Cu F.Paste F.Mask))
  (pad B7 smd circle (at -1.5 -2.75 180) (size 0.25 0.25) (layers F.Cu F.Paste F.Mask))
  (pad B5 smd circle (at -2 -2.75 180) (size 0.25 0.25) (layers F.Cu F.Paste F.Mask))
  (pad AC5 smd circle (at -2 2.75 180) (size 0.25 0.25) (layers F.Cu F.Paste F.Mask))
  (pad AC9 smd circle (at -1 2.75 180) (size 0.25 0.25) (layers F.Cu F.Paste F.Mask))
  (pad AC11 smd circle (at -0.5 2.75 180) (size 0.25 0.25) (layers F.Cu F.Paste F.Mask))
  (pad AC13 smd circle (at 0 2.75 180) (size 0.25 0.25) (layers F.Cu F.Paste F.Mask))
  (pad AC15 smd circle (at 0.5 2.75 180) (size 0.25 0.25) (layers F.Cu F.Paste F.Mask))
  (pad AC17 smd circle (at 1 2.75 180) (size 0.25 0.25) (layers F.Cu F.Paste F.Mask))
  (pad AC19 smd circle (at 1.5 2.75 180) (size 0.25 0.25) (layers F.Cu F.Paste F.Mask))
  (pad AD22 smd circle (at 2.25 3.25 180) (size 0.25 0.25) (layers F.Cu F.Paste F.Mask))
  (pad AD20 smd circle (at 1.75 3.25 180) (size 0.25 0.25) (layers F.Cu F.Paste F.Mask))
  (pad AD18 smd circle (at 1.25 3.25 180) (size 0.25 0.25) (layers F.Cu F.Paste F.Mask))
  (pad AD16 smd circle (at 0.75 3.25 180) (size 0.25 0.25) (layers F.Cu F.Paste F.Mask))
  (pad AD14 smd circle (at 0.25 3.25 180) (size 0.25 0.25) (layers F.Cu F.Paste F.Mask))
  (pad AD12 smd circle (at -0.25 3.25 180) (size 0.25 0.25) (layers F.Cu F.Paste F.Mask))
  (pad AD10 smd circle (at -0.75 3.25 180) (size 0.25 0.25) (layers F.Cu F.Paste F.Mask))
  (pad AD8 smd circle (at -1.25 3.25 180) (size 0.25 0.25) (layers F.Cu F.Paste F.Mask))
  (pad AD6 smd circle (at -1.75 3.25 180) (size 0.25 0.25) (layers F.Cu F.Paste F.Mask))
  (pad AD4 smd circle (at -2.25 3.25 180) (size 0.25 0.25) (layers F.Cu F.Paste F.Mask))
  (pad B1 smd circle (at -3.25 -2.75 180) (size 0.25 0.25) (layers F.Cu F.Paste F.Mask))
  (pad D2 smd circle (at -2.75 -2 180) (size 0.25 0.25) (layers F.Cu F.Paste F.Mask))
  (pad C1 smd circle (at -3.25 -2.25 180) (size 0.25 0.25) (layers F.Cu F.Paste F.Mask))
  (pad F2 smd circle (at -2.75 -1.5 180) (size 0.25 0.25) (layers F.Cu F.Paste F.Mask))
  (pad H2 smd circle (at -2.75 -1 180) (size 0.25 0.25) (layers F.Cu F.Paste F.Mask))
  (pad K2 smd circle (at -2.75 -0.5 180) (size 0.25 0.25) (layers F.Cu F.Paste F.Mask))
  (pad M2 smd circle (at -2.75 0 180) (size 0.25 0.25) (layers F.Cu F.Paste F.Mask))
  (pad P2 smd circle (at -2.75 0.5 180) (size 0.25 0.25) (layers F.Cu F.Paste F.Mask))
  (pad T2 smd circle (at -2.75 1 180) (size 0.25 0.25) (layers F.Cu F.Paste F.Mask))
  (pad G1 smd circle (at -3.25 -1.25 180) (size 0.25 0.25) (layers F.Cu F.Paste F.Mask))
  (pad J1 smd circle (at -3.25 -0.75 180) (size 0.25 0.25) (layers F.Cu F.Paste F.Mask))
  (pad L1 smd circle (at -3.25 -0.25 180) (size 0.25 0.25) (layers F.Cu F.Paste F.Mask))
  (pad N1 smd circle (at -3.25 0.25 180) (size 0.25 0.25) (layers F.Cu F.Paste F.Mask))
  (pad R1 smd circle (at -3.25 0.75 180) (size 0.25 0.25) (layers F.Cu F.Paste F.Mask))
  (pad U1 smd circle (at -3.25 1.25 180) (size 0.25 0.25) (layers F.Cu F.Paste F.Mask))
  (pad W1 smd circle (at -3.25 1.75 180) (size 0.25 0.25) (layers F.Cu F.Paste F.Mask))
  (pad Y2 smd circle (at -2.75 2 180) (size 0.25 0.25) (layers F.Cu F.Paste F.Mask))
  (pad AB2 smd circle (at -2.75 2.5 180) (size 0.25 0.25) (layers F.Cu F.Paste F.Mask))
  (pad AD2 smd circle (at -2.75 3.25 180) (size 0.25 0.25) (layers F.Cu F.Paste F.Mask))
  (pad AD23 smd circle (at 2.75 3.25 180) (size 0.25 0.25) (layers F.Cu F.Paste F.Mask))
  (pad AC21 smd circle (at 2 2.75 180) (size 0.25 0.25) (layers F.Cu F.Paste F.Mask))
  (pad B3 smd circle (at -2.5 -2.75 180) (size 0.25 0.25) (layers F.Cu F.Paste F.Mask))
  (pad A8 smd circle (at -1.25 -3.25 180) (size 0.25 0.25) (layers F.Cu F.Paste F.Mask))
  (pad D23 smd circle (at 2.75 -2 180) (size 0.25 0.25) (layers F.Cu F.Paste F.Mask))
  (pad B24 smd circle (at 3.25 -2.75 180) (size 0.25 0.25) (layers F.Cu F.Paste F.Mask))
  (pad EP smd rect (at 0 0 180) (size 4.85 4.85) (layers F.Cu F.Mask))
  (pad "" smd rect (at -1.2125 -1.2125 180) (size 2 2) (layers F.Paste))
  (pad "" smd rect (at 1.2125 -1.2125 180) (size 2 2) (layers F.Paste))
  (pad "" smd rect (at -1.2125 1.2125 180) (size 2 2) (layers F.Paste))
  (pad "" smd rect (at 1.2125 1.2125 180) (size 2 2) (layers F.Paste)))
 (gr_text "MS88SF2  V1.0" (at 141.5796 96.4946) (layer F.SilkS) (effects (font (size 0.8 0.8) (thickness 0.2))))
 (gr_line (start 148.3614 90.4494) (end 148.3868 113.6396) (layer Edge.Cuts) (width 0.05))
 (gr_line (start 148.3868 113.6396) (end 130.9624 113.6396) (layer Edge.Cuts) (width 0.05))
 (gr_line (start 130.937 90.4494) (end 148.3614 90.4494) (layer Edge.Cuts) (width 0.05))
 (gr_line (start 130.937 90.4494) (end 130.9624 113.6396) (layer Edge.Cuts) (width 0.05))
 (segment (start 133.35 92.075) (end 135.89 92.075) (width 0.508) (layer F.Cu) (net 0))
 (segment (start 135.89 92.075) (end 135.89 97.155) (width 0.508) (layer F.Cu) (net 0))
 (segment (start 135.89 92.075) (end 139.065 92.075) (width 0.508) (layer F.Cu) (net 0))
 (segment (start 139.065 92.075) (end 139.065 95.25) (width 0.508) (layer F.Cu) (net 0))
 (segment (start 139.065 95.25) (end 141.605 95.25) (width 0.508) (layer F.Cu) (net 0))
 (segment (start 141.605 95.25) (end 141.605 92.075) (width 0.508) (layer F.Cu) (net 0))
 (segment (start 141.605 92.075) (end 144.145 92.075) (width 0.508) (layer F.Cu) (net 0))
 (segment (start 144.145 92.075) (end 144.145 95.25) (width 0.508) (layer F.Cu) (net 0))
 (segment (start 144.145 95.25) (end 146.685 95.25) (width 0.508) (layer F.Cu) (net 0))
 (segment (start 146.685 95.25) (end 146.685 91.44) (width 0.508) (layer F.Cu) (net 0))
 (segment (start 133.477 96.774) (end 133.477 92.456) (width 1.27) (layer F.Cu) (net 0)))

